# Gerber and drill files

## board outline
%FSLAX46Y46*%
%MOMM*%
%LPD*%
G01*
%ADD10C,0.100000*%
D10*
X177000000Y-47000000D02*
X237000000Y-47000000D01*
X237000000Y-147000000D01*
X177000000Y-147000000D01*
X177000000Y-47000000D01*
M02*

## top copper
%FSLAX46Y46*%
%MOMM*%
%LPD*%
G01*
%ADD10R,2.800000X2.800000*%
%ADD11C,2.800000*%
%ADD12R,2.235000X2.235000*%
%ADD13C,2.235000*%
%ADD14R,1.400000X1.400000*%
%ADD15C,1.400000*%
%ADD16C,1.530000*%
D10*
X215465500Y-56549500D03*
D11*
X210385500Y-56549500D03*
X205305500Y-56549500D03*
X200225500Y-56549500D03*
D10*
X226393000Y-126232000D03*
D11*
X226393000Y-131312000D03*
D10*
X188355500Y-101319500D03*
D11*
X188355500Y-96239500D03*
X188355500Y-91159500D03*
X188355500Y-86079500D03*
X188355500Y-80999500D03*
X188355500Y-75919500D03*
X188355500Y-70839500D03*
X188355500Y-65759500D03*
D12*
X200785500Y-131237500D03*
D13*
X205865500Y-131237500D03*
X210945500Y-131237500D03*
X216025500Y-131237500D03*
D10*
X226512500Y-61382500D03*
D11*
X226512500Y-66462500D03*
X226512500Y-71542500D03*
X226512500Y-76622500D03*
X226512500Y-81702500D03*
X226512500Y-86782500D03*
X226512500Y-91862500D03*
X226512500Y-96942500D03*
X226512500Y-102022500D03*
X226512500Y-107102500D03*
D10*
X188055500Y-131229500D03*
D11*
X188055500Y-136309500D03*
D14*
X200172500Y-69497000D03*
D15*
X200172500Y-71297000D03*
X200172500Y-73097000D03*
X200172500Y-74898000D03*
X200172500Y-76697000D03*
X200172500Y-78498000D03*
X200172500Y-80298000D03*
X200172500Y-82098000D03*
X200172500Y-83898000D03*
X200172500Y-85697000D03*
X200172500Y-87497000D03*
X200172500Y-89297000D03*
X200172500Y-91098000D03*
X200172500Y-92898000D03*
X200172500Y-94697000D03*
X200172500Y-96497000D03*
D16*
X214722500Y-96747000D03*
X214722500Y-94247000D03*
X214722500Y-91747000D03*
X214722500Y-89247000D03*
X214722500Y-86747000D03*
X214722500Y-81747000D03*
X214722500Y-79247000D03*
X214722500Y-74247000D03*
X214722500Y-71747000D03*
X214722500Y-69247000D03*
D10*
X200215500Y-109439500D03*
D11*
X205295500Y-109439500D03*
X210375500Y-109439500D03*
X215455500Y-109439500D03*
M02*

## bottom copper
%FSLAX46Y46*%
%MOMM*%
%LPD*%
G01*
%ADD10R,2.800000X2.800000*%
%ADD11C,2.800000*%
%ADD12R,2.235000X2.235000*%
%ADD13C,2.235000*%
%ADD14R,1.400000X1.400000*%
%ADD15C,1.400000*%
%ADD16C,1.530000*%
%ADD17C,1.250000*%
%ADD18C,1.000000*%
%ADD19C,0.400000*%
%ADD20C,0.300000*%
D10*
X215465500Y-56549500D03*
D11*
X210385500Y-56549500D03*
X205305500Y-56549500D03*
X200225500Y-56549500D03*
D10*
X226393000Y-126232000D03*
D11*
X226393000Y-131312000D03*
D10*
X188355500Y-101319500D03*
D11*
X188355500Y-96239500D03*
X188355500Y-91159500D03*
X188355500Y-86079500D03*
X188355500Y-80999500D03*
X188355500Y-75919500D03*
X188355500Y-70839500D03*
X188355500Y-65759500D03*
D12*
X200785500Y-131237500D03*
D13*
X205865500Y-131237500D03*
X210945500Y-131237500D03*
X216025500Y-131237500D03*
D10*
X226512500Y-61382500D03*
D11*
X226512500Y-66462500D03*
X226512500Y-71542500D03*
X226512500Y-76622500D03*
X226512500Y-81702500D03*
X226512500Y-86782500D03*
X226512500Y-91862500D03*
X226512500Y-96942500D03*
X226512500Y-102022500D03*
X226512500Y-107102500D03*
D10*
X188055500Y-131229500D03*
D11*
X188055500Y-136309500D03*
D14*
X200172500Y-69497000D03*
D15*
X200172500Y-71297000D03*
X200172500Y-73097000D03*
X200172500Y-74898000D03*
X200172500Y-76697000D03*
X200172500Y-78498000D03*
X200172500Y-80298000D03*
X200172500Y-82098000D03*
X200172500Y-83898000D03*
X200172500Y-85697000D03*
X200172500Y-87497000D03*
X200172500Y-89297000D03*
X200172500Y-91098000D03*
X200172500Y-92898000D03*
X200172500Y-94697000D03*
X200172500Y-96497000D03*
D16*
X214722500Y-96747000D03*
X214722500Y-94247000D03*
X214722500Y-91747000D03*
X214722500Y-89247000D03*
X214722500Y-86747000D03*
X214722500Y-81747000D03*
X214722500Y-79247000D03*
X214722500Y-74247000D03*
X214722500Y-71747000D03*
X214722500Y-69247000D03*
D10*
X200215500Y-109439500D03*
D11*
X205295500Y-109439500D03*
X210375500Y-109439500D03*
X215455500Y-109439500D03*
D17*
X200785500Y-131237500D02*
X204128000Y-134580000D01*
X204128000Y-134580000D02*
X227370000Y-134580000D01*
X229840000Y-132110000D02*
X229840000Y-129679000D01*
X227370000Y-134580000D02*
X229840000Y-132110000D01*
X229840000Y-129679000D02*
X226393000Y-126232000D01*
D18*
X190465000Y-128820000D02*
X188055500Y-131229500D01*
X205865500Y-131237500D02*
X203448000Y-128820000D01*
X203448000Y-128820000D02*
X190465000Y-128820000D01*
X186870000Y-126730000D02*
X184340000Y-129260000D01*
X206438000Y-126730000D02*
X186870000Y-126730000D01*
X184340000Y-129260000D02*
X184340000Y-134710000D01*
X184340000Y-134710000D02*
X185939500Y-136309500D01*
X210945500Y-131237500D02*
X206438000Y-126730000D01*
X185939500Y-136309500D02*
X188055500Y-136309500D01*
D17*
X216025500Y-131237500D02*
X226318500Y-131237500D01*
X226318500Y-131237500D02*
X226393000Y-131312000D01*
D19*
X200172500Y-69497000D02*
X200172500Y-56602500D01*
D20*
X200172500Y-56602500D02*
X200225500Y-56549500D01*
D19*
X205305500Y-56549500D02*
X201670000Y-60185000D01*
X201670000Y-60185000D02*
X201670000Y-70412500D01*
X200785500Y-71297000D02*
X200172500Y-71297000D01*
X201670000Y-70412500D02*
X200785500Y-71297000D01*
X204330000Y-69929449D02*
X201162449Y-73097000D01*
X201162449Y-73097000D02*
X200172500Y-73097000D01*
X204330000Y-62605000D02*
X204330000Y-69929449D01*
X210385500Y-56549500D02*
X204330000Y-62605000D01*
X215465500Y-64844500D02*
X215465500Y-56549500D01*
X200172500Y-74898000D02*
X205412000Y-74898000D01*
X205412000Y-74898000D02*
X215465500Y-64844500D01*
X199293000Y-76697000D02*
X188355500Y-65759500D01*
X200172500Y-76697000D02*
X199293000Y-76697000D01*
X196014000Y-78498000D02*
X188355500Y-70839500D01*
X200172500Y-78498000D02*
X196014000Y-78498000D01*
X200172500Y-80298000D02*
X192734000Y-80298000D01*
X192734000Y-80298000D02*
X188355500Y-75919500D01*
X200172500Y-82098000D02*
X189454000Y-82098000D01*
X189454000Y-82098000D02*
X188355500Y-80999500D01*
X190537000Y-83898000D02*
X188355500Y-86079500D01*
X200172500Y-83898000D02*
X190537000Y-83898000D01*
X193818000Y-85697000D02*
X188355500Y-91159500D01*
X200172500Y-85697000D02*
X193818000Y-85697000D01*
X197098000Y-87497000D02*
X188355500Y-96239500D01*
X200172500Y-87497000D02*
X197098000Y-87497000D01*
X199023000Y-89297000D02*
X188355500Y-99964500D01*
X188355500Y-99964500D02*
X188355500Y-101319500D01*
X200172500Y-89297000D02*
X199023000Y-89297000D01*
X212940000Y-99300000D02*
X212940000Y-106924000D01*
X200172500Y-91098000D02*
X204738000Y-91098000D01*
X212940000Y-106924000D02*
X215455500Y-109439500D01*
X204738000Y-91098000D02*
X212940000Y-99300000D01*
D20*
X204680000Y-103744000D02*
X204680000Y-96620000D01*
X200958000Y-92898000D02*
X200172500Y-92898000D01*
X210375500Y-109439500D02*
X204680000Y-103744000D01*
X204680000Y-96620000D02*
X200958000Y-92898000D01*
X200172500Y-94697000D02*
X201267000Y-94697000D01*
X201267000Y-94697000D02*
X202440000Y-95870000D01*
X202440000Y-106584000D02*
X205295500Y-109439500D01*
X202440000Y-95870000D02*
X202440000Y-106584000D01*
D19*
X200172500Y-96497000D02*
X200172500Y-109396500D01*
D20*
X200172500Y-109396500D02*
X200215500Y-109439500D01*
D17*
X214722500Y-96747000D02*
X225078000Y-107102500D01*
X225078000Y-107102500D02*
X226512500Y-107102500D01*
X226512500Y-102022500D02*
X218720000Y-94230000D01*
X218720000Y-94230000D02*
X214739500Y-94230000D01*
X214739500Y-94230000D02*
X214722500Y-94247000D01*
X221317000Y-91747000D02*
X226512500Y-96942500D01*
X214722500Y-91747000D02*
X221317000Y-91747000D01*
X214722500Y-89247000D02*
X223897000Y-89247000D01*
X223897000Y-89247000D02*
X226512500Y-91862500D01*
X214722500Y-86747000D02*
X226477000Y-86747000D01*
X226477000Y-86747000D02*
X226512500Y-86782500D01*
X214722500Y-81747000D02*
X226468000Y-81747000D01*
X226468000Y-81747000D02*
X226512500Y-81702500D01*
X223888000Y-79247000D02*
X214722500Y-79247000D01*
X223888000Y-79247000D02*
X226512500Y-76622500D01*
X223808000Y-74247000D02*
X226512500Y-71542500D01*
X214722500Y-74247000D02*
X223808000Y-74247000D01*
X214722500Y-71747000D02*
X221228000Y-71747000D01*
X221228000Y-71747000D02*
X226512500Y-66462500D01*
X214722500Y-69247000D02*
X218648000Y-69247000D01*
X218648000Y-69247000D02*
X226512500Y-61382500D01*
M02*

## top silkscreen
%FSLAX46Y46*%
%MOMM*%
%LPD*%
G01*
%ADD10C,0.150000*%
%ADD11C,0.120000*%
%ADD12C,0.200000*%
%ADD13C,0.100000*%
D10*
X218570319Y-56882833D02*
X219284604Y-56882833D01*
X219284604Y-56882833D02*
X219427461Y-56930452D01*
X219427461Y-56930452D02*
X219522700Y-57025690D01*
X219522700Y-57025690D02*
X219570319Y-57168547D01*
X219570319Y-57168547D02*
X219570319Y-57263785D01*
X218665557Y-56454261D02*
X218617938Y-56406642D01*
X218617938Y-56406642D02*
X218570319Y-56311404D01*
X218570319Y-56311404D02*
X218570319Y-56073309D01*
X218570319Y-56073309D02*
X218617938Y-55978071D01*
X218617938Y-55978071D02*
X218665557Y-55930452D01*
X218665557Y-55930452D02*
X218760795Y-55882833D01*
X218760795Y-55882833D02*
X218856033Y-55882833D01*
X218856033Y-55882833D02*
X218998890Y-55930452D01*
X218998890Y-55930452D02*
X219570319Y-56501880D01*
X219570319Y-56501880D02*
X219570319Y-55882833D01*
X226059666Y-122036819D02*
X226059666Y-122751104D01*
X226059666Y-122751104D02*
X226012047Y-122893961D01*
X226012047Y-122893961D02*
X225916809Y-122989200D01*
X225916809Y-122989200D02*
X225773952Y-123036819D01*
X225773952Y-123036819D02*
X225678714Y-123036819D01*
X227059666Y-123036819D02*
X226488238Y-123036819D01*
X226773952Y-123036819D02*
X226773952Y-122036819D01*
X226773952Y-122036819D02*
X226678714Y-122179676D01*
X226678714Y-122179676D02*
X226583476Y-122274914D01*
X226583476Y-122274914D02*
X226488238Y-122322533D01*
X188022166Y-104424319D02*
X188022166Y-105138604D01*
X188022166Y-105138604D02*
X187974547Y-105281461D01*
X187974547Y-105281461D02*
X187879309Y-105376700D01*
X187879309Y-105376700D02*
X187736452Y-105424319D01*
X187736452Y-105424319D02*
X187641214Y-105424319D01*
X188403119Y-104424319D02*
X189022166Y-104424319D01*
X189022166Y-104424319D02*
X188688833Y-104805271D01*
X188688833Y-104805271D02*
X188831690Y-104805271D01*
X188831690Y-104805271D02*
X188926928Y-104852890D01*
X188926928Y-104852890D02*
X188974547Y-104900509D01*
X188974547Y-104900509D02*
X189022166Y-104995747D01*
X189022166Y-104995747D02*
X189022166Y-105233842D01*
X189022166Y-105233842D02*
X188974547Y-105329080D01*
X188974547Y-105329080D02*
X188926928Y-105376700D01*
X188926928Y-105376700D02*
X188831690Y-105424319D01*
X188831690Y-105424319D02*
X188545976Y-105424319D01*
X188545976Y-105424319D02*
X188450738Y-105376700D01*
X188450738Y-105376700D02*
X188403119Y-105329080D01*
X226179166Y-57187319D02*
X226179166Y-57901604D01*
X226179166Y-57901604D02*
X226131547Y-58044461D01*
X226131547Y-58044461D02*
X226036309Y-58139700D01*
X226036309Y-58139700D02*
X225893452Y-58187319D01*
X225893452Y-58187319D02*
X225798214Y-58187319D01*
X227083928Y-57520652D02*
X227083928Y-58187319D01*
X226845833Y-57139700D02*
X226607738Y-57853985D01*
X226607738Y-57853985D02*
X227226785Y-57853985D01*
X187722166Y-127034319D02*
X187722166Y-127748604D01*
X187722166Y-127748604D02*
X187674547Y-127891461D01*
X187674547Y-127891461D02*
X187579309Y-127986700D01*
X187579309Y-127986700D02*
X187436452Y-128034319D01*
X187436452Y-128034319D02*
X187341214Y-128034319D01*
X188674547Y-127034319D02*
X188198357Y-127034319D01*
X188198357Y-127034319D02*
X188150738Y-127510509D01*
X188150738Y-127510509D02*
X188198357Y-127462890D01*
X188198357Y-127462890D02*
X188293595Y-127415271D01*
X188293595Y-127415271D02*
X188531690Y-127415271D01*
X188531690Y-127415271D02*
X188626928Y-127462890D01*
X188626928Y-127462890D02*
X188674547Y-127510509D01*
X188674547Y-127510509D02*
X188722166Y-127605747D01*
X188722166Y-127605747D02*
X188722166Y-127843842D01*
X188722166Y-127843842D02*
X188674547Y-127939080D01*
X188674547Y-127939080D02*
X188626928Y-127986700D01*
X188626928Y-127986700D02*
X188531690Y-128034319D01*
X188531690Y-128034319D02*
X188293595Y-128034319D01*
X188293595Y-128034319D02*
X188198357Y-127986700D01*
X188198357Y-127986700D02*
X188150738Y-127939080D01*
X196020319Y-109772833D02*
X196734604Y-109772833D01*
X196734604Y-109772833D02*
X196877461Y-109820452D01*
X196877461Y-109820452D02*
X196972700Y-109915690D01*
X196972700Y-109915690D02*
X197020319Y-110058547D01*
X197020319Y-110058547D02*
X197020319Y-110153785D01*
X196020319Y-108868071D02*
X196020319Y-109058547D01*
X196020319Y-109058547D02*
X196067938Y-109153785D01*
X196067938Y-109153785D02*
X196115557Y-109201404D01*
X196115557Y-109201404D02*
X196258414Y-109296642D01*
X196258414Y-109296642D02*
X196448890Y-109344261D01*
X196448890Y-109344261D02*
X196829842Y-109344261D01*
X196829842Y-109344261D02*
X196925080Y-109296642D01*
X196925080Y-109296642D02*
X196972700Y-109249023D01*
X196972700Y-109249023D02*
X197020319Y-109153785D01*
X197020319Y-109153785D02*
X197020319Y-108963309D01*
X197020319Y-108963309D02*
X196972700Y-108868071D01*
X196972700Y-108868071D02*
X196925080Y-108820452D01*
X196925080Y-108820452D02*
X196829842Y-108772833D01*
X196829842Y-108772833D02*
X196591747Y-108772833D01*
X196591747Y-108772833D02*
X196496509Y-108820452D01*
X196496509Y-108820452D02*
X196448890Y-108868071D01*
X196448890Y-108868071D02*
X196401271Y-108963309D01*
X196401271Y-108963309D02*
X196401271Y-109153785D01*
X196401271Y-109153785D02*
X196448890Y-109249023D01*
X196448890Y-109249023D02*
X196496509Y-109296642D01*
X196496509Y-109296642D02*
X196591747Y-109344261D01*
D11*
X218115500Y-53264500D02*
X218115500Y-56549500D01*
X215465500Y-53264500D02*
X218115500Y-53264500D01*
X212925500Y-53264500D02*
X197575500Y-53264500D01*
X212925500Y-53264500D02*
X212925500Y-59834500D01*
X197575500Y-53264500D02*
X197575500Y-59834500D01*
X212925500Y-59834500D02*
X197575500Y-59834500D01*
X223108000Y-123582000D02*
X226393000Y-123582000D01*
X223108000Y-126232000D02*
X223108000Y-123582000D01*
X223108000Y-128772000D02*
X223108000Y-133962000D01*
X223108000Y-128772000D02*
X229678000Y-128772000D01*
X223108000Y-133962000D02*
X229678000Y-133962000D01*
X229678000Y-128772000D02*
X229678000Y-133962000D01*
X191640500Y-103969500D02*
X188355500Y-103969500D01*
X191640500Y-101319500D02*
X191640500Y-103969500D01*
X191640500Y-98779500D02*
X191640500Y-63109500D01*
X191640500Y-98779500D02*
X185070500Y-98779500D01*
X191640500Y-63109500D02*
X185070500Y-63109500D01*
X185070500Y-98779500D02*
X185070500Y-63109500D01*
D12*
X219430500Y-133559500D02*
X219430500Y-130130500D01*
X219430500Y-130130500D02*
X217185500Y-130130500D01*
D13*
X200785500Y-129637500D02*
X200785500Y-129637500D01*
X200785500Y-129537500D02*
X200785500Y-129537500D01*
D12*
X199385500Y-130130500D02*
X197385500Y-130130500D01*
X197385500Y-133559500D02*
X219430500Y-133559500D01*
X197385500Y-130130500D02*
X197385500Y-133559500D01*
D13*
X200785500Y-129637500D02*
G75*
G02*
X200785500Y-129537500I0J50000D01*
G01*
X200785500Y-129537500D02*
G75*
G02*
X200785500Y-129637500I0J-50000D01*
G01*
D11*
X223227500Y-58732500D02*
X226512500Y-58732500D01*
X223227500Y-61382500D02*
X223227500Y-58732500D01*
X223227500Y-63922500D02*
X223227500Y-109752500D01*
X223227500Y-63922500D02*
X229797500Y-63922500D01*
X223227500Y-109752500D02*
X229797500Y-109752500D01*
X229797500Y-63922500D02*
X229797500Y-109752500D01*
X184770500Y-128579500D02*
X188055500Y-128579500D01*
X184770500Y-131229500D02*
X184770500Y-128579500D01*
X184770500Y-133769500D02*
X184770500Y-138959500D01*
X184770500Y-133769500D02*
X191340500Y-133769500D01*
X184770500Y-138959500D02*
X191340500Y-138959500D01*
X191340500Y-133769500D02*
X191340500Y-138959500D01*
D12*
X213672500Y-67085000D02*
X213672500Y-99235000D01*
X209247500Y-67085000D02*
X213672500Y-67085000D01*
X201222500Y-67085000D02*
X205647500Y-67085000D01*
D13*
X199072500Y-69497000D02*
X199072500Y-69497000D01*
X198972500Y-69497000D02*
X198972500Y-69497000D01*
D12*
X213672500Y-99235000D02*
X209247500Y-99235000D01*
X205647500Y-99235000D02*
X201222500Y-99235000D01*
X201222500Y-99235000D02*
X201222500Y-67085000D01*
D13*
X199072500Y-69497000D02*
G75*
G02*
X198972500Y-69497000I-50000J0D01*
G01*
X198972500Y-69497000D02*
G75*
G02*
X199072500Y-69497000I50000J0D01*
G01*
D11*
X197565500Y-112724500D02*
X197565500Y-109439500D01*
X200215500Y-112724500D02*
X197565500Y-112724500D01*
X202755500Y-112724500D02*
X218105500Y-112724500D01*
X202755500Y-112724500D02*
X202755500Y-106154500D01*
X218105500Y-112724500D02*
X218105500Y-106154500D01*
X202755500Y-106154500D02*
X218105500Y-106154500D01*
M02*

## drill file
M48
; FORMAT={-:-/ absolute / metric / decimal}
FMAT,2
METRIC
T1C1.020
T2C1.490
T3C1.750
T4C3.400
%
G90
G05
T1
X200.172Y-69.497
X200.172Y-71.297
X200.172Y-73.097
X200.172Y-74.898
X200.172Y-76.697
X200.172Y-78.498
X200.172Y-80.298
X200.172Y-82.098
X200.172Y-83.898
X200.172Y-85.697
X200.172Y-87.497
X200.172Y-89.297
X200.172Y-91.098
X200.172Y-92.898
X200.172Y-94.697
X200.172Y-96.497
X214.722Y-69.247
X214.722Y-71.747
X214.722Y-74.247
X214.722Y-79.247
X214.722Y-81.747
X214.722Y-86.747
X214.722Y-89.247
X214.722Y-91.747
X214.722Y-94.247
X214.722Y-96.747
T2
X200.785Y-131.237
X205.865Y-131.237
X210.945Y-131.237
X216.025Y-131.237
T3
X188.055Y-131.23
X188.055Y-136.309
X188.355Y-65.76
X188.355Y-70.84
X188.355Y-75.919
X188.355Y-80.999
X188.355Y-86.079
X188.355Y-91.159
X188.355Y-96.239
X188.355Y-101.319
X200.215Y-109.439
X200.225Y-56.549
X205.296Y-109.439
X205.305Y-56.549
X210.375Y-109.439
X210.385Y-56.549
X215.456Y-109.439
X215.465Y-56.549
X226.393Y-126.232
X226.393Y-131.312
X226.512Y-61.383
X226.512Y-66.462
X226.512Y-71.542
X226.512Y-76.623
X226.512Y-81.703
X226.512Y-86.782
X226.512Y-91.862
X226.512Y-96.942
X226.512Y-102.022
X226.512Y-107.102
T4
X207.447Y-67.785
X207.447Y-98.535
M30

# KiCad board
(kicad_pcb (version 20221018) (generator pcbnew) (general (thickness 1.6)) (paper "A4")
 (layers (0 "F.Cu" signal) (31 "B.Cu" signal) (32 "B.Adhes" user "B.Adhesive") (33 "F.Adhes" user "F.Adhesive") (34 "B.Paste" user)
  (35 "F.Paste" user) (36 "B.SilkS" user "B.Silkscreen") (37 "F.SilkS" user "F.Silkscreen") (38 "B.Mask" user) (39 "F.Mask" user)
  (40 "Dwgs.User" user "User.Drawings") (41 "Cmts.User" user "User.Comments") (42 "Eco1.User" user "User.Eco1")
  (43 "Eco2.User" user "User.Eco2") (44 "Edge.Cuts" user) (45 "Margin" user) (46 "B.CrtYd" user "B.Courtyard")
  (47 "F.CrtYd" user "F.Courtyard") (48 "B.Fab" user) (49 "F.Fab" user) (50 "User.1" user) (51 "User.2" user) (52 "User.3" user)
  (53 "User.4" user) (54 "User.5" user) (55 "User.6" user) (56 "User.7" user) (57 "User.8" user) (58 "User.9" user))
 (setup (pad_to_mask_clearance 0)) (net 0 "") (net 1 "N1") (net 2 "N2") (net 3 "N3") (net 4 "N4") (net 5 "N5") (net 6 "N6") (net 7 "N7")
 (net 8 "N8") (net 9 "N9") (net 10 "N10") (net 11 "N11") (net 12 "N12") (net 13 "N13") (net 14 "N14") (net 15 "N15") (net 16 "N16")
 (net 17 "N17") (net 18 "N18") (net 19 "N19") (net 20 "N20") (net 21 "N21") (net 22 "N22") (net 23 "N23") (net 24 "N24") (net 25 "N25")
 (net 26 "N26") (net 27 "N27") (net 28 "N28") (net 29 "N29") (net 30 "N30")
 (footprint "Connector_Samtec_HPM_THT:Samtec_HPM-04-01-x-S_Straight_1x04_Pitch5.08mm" (layer "F.Cu") (at 215.4655 56.5495 -90)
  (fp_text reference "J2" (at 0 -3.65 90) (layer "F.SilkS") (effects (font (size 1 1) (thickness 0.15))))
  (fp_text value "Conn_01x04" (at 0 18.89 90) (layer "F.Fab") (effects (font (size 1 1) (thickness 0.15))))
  (fp_line (start -3.285 -2.65) (end 0 -2.65) (stroke (width 0.12) (type solid)) (layer "F.SilkS"))
  (fp_line (start -3.285 0) (end -3.285 -2.65) (stroke (width 0.12) (type solid)) (layer "F.SilkS"))
  (fp_line (start -3.285 2.54) (end -3.285 17.89) (stroke (width 0.12) (type solid)) (layer "F.SilkS"))
  (fp_line (start -3.285 2.54) (end 3.285 2.54) (stroke (width 0.12) (type solid)) (layer "F.SilkS"))
  (fp_line (start -3.285 17.89) (end 3.285 17.89) (stroke (width 0.12) (type solid)) (layer "F.SilkS"))
  (fp_line (start 3.285 2.54) (end 3.285 17.89) (stroke (width 0.12) (type solid)) (layer "F.SilkS"))
  (pad "1" thru_hole rect (at 0 0 270) (size 2.8 2.8) (drill 1.75) (layers "*.Cu" "*.Mask") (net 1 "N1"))
  (pad "2" thru_hole circle (at 0 5.08 270) (size 2.8 2.8) (drill 1.75) (layers "*.Cu" "*.Mask") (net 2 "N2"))
  (pad "3" thru_hole circle (at 0 10.16 270) (size 2.8 2.8) (drill 1.75) (layers "*.Cu" "*.Mask") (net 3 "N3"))
  (pad "4" thru_hole circle (at 0 15.24 270) (size 2.8 2.8) (drill 1.75) (layers "*.Cu" "*.Mask") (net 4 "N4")))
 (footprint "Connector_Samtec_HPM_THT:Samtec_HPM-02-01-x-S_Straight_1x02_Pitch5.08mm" (layer "F.Cu") (at 226.393 126.232)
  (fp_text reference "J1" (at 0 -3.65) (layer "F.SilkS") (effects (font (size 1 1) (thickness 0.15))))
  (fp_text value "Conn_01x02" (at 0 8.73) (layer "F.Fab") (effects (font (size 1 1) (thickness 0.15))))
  (fp_line (start -3.285 -2.65) (end 0 -2.65) (stroke (width 0.12) (type solid)) (layer "F.SilkS"))
  (fp_line (start -3.285 0) (end -3.285 -2.65) (stroke (width 0.12) (type solid)) (layer "F.SilkS"))
  (fp_line (start -3.285 2.54) (end -3.285 7.73) (stroke (width 0.12) (type solid)) (layer "F.SilkS"))
  (fp_line (start -3.285 2.54) (end 3.285 2.54) (stroke (width 0.12) (type solid)) (layer "F.SilkS"))
  (fp_line (start -3.285 7.73) (end 3.285 7.73) (stroke (width 0.12) (type solid)) (layer "F.SilkS"))
  (fp_line (start 3.285 2.54) (end 3.285 7.73) (stroke (width 0.12) (type solid)) (layer "F.SilkS"))
  (pad "1" thru_hole rect (at 0 0) (size 2.8 2.8) (drill 1.75) (layers "*.Cu" "*.Mask") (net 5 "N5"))
  (pad "2" thru_hole circle (at 0 5.08) (size 2.8 2.8) (drill 1.75) (layers "*.Cu" "*.Mask") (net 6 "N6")))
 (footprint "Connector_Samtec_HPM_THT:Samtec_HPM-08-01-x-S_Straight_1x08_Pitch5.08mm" (layer "F.Cu") (at 188.3555 101.3195 180)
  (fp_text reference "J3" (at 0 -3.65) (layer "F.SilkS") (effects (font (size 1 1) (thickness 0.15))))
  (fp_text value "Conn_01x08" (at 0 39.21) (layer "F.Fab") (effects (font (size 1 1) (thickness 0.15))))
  (fp_line (start -3.285 -2.65) (end 0 -2.65) (stroke (width 0.12) (type solid)) (layer "F.SilkS"))
  (fp_line (start -3.285 0) (end -3.285 -2.65) (stroke (width 0.12) (type solid)) (layer "F.SilkS"))
  (fp_line (start -3.285 2.54) (end -3.285 38.21) (stroke (width 0.12) (type solid)) (layer "F.SilkS"))
  (fp_line (start -3.285 2.54) (end 3.285 2.54) (stroke (width 0.12) (type solid)) (layer "F.SilkS"))
  (fp_line (start -3.285 38.21) (end 3.285 38.21) (stroke (width 0.12) (type solid)) (layer "F.SilkS"))
  (fp_line (start 3.285 2.54) (end 3.285 38.21) (stroke (width 0.12) (type solid)) (layer "F.SilkS"))
  (pad "1" thru_hole rect (at 0 0 180) (size 2.8 2.8) (drill 1.75) (layers "*.Cu" "*.Mask") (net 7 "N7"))
  (pad "2" thru_hole circle (at 0 5.08 180) (size 2.8 2.8) (drill 1.75) (layers "*.Cu" "*.Mask") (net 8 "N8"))
  (pad "3" thru_hole circle (at 0 10.16 180) (size 2.8 2.8) (drill 1.75) (layers "*.Cu" "*.Mask") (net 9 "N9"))
  (pad "4" thru_hole circle (at 0 15.24 180) (size 2.8 2.8) (drill 1.75) (layers "*.Cu" "*.Mask") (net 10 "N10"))
  (pad "5" thru_hole circle (at 0 20.32 180) (size 2.8 2.8) (drill 1.75) (layers "*.Cu" "*.Mask") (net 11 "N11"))
  (pad "6" thru_hole circle (at 0 25.4 180) (size 2.8 2.8) (drill 1.75) (layers "*.Cu" "*.Mask") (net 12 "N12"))
  (pad "7" thru_hole circle (at 0 30.48 180) (size 2.8 2.8) (drill 1.75) (layers "*.Cu" "*.Mask") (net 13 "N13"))
  (pad "8" thru_hole circle (at 0 35.56 180) (size 2.8 2.8) (drill 1.75) (layers "*.Cu" "*.Mask") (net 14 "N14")))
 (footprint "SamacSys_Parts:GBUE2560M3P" (layer "F.Cu") (at 200.7855 131.2375 180)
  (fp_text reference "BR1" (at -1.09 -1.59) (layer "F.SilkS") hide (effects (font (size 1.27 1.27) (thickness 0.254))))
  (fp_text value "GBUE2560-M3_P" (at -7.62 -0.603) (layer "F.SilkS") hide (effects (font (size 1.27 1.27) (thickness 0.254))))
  (fp_line (start -18.645 -2.322) (end -18.645 1.107) (stroke (width 0.2) (type solid)) (layer "F.SilkS"))
  (fp_line (start -18.645 1.107) (end -16.4 1.107) (stroke (width 0.2) (type solid)) (layer "F.SilkS"))
  (fp_line (start 0 1.6) (end 0 1.6) (stroke (width 0.1) (type solid)) (layer "F.SilkS"))
  (fp_line (start 0 1.7) (end 0 1.7) (stroke (width 0.1) (type solid)) (layer "F.SilkS"))
  (fp_line (start 1.4 1.107) (end 3.4 1.107) (stroke (width 0.2) (type solid)) (layer "F.SilkS"))
  (fp_line (start 3.4 -2.322) (end -18.645 -2.322) (stroke (width 0.2) (type solid)) (layer "F.SilkS"))
  (fp_line (start 3.4 1.107) (end 3.4 -2.322) (stroke (width 0.2) (type solid)) (layer "F.SilkS"))
  (fp_arc (start 0 1.6) (mid 0.05 1.65) (end 0 1.7) (stroke (width 0.1) (type solid)) (layer "F.SilkS"))
  (fp_arc (start 0 1.7) (mid -0.05 1.65) (end 0 1.6) (stroke (width 0.1) (type solid)) (layer "F.SilkS"))
  (pad "1" thru_hole rect (at 0 0 180) (size 2.235 2.235) (drill 1.49) (layers "*.Cu" "*.Mask") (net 5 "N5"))
  (pad "2" thru_hole circle (at -5.08 0 180) (size 2.235 2.235) (drill 1.49) (layers "*.Cu" "*.Mask") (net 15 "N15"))
  (pad "3" thru_hole circle (at -10.16 0 180) (size 2.235 2.235) (drill 1.49) (layers "*.Cu" "*.Mask") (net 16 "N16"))
  (pad "4" thru_hole circle (at -15.24 0 180) (size 2.235 2.235) (drill 1.49) (layers "*.Cu" "*.Mask") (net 6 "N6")))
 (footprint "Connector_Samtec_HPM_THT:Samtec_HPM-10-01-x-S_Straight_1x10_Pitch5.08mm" (layer "F.Cu") (at 226.5125 61.3825)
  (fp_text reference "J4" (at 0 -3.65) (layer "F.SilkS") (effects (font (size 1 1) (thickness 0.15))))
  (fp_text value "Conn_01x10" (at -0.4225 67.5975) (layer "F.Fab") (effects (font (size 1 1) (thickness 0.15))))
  (fp_line (start -3.285 -2.65) (end 0 -2.65) (stroke (width 0.12) (type solid)) (layer "F.SilkS"))
  (fp_line (start -3.285 0) (end -3.285 -2.65) (stroke (width 0.12) (type solid)) (layer "F.SilkS"))
  (fp_line (start -3.285 2.54) (end -3.285 48.37) (stroke (width 0.12) (type solid)) (layer "F.SilkS"))
  (fp_line (start -3.285 2.54) (end 3.285 2.54) (stroke (width 0.12) (type solid)) (layer "F.SilkS"))
  (fp_line (start -3.285 48.37) (end 3.285 48.37) (stroke (width 0.12) (type solid)) (layer "F.SilkS"))
  (fp_line (start 3.285 2.54) (end 3.285 48.37) (stroke (width 0.12) (type solid)) (layer "F.SilkS"))
  (pad "1" thru_hole rect (at 0 0) (size 2.8 2.8) (drill 1.75) (layers "*.Cu" "*.Mask") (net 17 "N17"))
  (pad "2" thru_hole circle (at 0 5.08) (size 2.8 2.8) (drill 1.75) (layers "*.Cu" "*.Mask") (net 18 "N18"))
  (pad "3" thru_hole circle (at 0 10.16) (size 2.8 2.8) (drill 1.75) (layers "*.Cu" "*.Mask") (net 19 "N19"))
  (pad "4" thru_hole circle (at 0 15.24) (size 2.8 2.8) (drill 1.75) (layers "*.Cu" "*.Mask") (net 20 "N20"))
  (pad "5" thru_hole circle (at 0 20.32) (size 2.8 2.8) (drill 1.75) (layers "*.Cu" "*.Mask") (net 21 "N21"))
  (pad "6" thru_hole circle (at 0 25.4) (size 2.8 2.8) (drill 1.75) (layers "*.Cu" "*.Mask") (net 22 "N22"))
  (pad "7" thru_hole circle (at 0 30.48) (size 2.8 2.8) (drill 1.75) (layers "*.Cu" "*.Mask") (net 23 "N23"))
  (pad "8" thru_hole circle (at 0 35.56) (size 2.8 2.8) (drill 1.75) (layers "*.Cu" "*.Mask") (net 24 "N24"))
  (pad "9" thru_hole circle (at 0 40.64) (size 2.8 2.8) (drill 1.75) (layers "*.Cu" "*.Mask") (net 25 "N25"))
  (pad "10" thru_hole circle (at 0 45.72) (size 2.8 2.8) (drill 1.75) (layers "*.Cu" "*.Mask") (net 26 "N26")))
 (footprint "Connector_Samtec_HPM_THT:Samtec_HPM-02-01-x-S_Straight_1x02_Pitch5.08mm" (layer "F.Cu") (at 188.0555 131.2295)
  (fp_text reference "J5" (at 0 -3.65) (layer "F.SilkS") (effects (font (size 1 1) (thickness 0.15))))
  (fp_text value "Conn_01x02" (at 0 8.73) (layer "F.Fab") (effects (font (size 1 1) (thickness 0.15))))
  (fp_line (start -3.285 -2.65) (end 0 -2.65) (stroke (width 0.12) (type solid)) (layer "F.SilkS"))
  (fp_line (start -3.285 0) (end -3.285 -2.65) (stroke (width 0.12) (type solid)) (layer "F.SilkS"))
  (fp_line (start -3.285 2.54) (end -3.285 7.73) (stroke (width 0.12) (type solid)) (layer "F.SilkS"))
  (fp_line (start -3.285 2.54) (end 3.285 2.54) (stroke (width 0.12) (type solid)) (layer "F.SilkS"))
  (fp_line (start -3.285 7.73) (end 3.285 7.73) (stroke (width 0.12) (type solid)) (layer "F.SilkS"))
  (fp_line (start 3.285 2.54) (end 3.285 7.73) (stroke (width 0.12) (type solid)) (layer "F.SilkS"))
  (pad "1" thru_hole rect (at 0 0) (size 2.8 2.8) (drill 1.75) (layers "*.Cu" "*.Mask") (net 15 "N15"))
  (pad "2" thru_hole circle (at 0 5.08) (size 2.8 2.8) (drill 1.75) (layers "*.Cu" "*.Mask") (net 16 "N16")))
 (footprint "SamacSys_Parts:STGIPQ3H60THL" (layer "F.Cu") (at 200.1725 69.497 -90)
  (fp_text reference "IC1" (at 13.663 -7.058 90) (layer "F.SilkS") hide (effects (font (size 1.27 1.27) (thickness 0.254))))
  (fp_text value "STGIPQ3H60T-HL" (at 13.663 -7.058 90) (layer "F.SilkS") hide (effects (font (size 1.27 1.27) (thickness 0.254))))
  (fp_line (start -2.412 -13.5) (end 29.738 -13.5) (stroke (width 0.2) (type solid)) (layer "F.SilkS"))
  (fp_line (start -2.412 -9.075) (end -2.412 -13.5) (stroke (width 0.2) (type solid)) (layer "F.SilkS"))
  (fp_line (start -2.412 -1.05) (end -2.412 -5.475) (stroke (width 0.2) (type solid)) (layer "F.SilkS"))
  (fp_line (start 0 1.1) (end 0 1.1) (stroke (width 0.1) (type solid)) (layer "F.SilkS"))
  (fp_line (start 0 1.2) (end 0 1.2) (stroke (width 0.1) (type solid)) (layer "F.SilkS"))
  (fp_line (start 29.738 -13.5) (end 29.738 -9.075) (stroke (width 0.2) (type solid)) (layer "F.SilkS"))
  (fp_line (start 29.738 -5.475) (end 29.738 -1.05) (stroke (width 0.2) (type solid)) (layer "F.SilkS"))
  (fp_line (start 29.738 -1.05) (end -2.412 -1.05) (stroke (width 0.2) (type solid)) (layer "F.SilkS"))
  (fp_arc (start 0 1.1) (mid 0.05 1.15) (end 0 1.2) (stroke (width 0.1) (type solid)) (layer "F.SilkS"))
  (fp_arc (start 0 1.2) (mid -0.05 1.15) (end 0 1.1) (stroke (width 0.1) (type solid)) (layer "F.SilkS"))
  (pad "" np_thru_hole circle (at -1.712 -7.275 270) (size 3.4 3.4) (drill 3.4) (layers "*.Cu" "*.Mask"))
  (pad "" np_thru_hole circle (at 29.038 -7.275 270) (size 3.4 3.4) (drill 3.4) (layers "*.Cu" "*.Mask"))
  (pad "1" thru_hole rect (at 0 0 270) (size 1.4 1.4) (drill 1.02) (layers "*.Cu" "*.Mask") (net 4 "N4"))
  (pad "2" thru_hole circle (at 1.8 0 270) (size 1.4 1.4) (drill 1.02) (layers "*.Cu" "*.Mask") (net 3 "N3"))
  (pad "3" thru_hole circle (at 3.6 0 270) (size 1.4 1.4) (drill 1.02) (layers "*.Cu" "*.Mask") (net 2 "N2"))
  (pad "4" thru_hole circle (at 5.401 0 270) (size 1.4 1.4) (drill 1.02) (layers "*.Cu" "*.Mask") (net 1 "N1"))
  (pad "5" thru_hole circle (at 7.2 0 270) (size 1.4 1.4) (drill 1.02) (layers "*.Cu" "*.Mask") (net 14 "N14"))
  (pad "6" thru_hole circle (at 9.001 0 270) (size 1.4 1.4) (drill 1.02) (layers "*.Cu" "*.Mask") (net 13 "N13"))
  (pad "7" thru_hole circle (at 10.801 0 270) (size 1.4 1.4) (drill 1.02) (layers "*.Cu" "*.Mask") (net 12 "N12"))
  (pad "8" thru_hole circle (at 12.601 0 270) (size 1.4 1.4) (drill 1.02) (layers "*.Cu" "*.Mask") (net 11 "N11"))
  (pad "9" thru_hole circle (at 14.401 0 270) (size 1.4 1.4) (drill 1.02) (layers "*.Cu" "*.Mask") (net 10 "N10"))
  (pad "10" thru_hole circle (at 16.2 0 270) (size 1.4 1.4) (drill 1.02) (layers "*.Cu" "*.Mask") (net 9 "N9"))
  (pad "11" thru_hole circle (at 18 0 270) (size 1.4 1.4) (drill 1.02) (layers "*.Cu" "*.Mask") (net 8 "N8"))
  (pad "12" thru_hole circle (at 19.8 0 270) (size 1.4 1.4) (drill 1.02) (layers "*.Cu" "*.Mask") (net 7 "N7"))
  (pad "13" thru_hole circle (at 21.601 0 270) (size 1.4 1.4) (drill 1.02) (layers "*.Cu" "*.Mask") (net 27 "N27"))
  (pad "14" thru_hole circle (at 23.401 0 270) (size 1.4 1.4) (drill 1.02) (layers "*.Cu" "*.Mask") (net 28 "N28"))
  (pad "15" thru_hole circle (at 25.2 0 270) (size 1.4 1.4) (drill 1.02) (layers "*.Cu" "*.Mask") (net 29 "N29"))
  (pad "16" thru_hole circle (at 27 0 270) (size 1.4 1.4) (drill 1.02) (layers "*.Cu" "*.Mask") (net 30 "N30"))
  (pad "17" thru_hole circle (at 27.25 -14.55 270) (size 1.53 1.53) (drill 1.02) (layers "*.Cu" "*.Mask") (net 26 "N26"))
  (pad "18" thru_hole circle (at 24.75 -14.55 270) (size 1.53 1.53) (drill 1.02) (layers "*.Cu" "*.Mask") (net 25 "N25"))
  (pad "19" thru_hole circle (at 22.25 -14.55 270) (size 1.53 1.53) (drill 1.02) (layers "*.Cu" "*.Mask") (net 24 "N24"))
  (pad "20" thru_hole circle (at 19.75 -14.55 270) (size 1.53 1.53) (drill 1.02) (layers "*.Cu" "*.Mask") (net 23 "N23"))
  (pad "21" thru_hole circle (at 17.25 -14.55 270) (size 1.53 1.53) (drill 1.02) (layers "*.Cu" "*.Mask") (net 22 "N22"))
  (pad "22" thru_hole circle (at 12.25 -14.55 270) (size 1.53 1.53) (drill 1.02) (layers "*.Cu" "*.Mask") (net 21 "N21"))
  (pad "23" thru_hole circle (at 9.75 -14.55 270) (size 1.53 1.53) (drill 1.02) (layers "*.Cu" "*.Mask") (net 20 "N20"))
  (pad "24" thru_hole circle (at 4.75 -14.55 270) (size 1.53 1.53) (drill 1.02) (layers "*.Cu" "*.Mask") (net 19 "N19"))
  (pad "25" thru_hole circle (at 2.25 -14.55 270) (size 1.53 1.53) (drill 1.02) (layers "*.Cu" "*.Mask") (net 18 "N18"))
  (pad "26" thru_hole circle (at -0.25 -14.55 270) (size 1.53 1.53) (drill 1.02) (layers "*.Cu" "*.Mask") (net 17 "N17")))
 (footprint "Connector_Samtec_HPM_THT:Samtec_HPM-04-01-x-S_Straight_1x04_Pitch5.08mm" (layer "F.Cu") (at 200.2155 109.4395 90)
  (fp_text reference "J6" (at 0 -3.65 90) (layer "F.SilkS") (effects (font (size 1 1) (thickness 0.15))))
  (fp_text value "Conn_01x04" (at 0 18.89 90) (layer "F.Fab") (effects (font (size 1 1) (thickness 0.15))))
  (fp_line (start -3.285 -2.65) (end 0 -2.65) (stroke (width 0.12) (type solid)) (layer "F.SilkS"))
  (fp_line (start -3.285 0) (end -3.285 -2.65) (stroke (width 0.12) (type solid)) (layer "F.SilkS"))
  (fp_line (start -3.285 2.54) (end -3.285 17.89) (stroke (width 0.12) (type solid)) (layer "F.SilkS"))
  (fp_line (start -3.285 2.54) (end 3.285 2.54) (stroke (width 0.12) (type solid)) (layer "F.SilkS"))
  (fp_line (start -3.285 17.89) (end 3.285 17.89) (stroke (width 0.12) (type solid)) (layer "F.SilkS"))
  (fp_line (start 3.285 2.54) (end 3.285 17.89) (stroke (width 0.12) (type solid)) (layer "F.SilkS"))
  (pad "1" thru_hole rect (at 0 0 90) (size 2.8 2.8) (drill 1.75) (layers "*.Cu" "*.Mask") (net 30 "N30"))
  (pad "2" thru_hole circle (at 0 5.08 90) (size 2.8 2.8) (drill 1.75) (layers "*.Cu" "*.Mask") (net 29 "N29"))
  (pad "3" thru_hole circle (at 0 10.16 90) (size 2.8 2.8) (drill 1.75) (layers "*.Cu" "*.Mask") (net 28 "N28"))
  (pad "4" thru_hole circle (at 0 15.24 90) (size 2.8 2.8) (drill 1.75) (layers "*.Cu" "*.Mask") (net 27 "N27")))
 (gr_rect (start 177 47) (end 237 147) (stroke (width 0.1) (type default)) (fill none) (layer "Edge.Cuts"))
 (segment (start 200.7855 131.2375) (end 204.128 134.58) (width 1.25) (layer "B.Cu") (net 5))
 (segment (start 204.128 134.58) (end 227.37 134.58) (width 1.25) (layer "B.Cu") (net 5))
 (segment (start 229.84 132.11) (end 229.84 129.679) (width 1.25) (layer "B.Cu") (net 5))
 (segment (start 227.37 134.58) (end 229.84 132.11) (width 1.25) (layer "B.Cu") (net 5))
 (segment (start 229.84 129.679) (end 226.393 126.232) (width 1.25) (layer "B.Cu") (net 5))
 (segment (start 190.465 128.82) (end 188.0555 131.2295) (width 1) (layer "B.Cu") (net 15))
 (segment (start 205.8655 131.2375) (end 203.448 128.82) (width 1) (layer "B.Cu") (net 15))
 (segment (start 203.448 128.82) (end 190.465 128.82) (width 1) (layer "B.Cu") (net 15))
 (segment (start 186.87 126.73) (end 184.34 129.26) (width 1) (layer "B.Cu") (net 16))
 (segment (start 206.438 126.73) (end 186.87 126.73) (width 1) (layer "B.Cu") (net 16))
 (segment (start 184.34 129.26) (end 184.34 134.71) (width 1) (layer "B.Cu") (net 16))
 (segment (start 184.34 134.71) (end 185.9395 136.3095) (width 1) (layer "B.Cu") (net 16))
 (segment (start 210.9455 131.2375) (end 206.438 126.73) (width 1) (layer "B.Cu") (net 16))
 (segment (start 185.9395 136.3095) (end 188.0555 136.3095) (width 1) (layer "B.Cu") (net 16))
 (segment (start 216.0255 131.2375) (end 226.3185 131.2375) (width 1.25) (layer "B.Cu") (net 6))
 (segment (start 226.3185 131.2375) (end 226.393 131.312) (width 1.25) (layer "B.Cu") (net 6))
 (segment (start 200.1725 69.497) (end 200.1725 56.6025) (width 0.4) (layer "B.Cu") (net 4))
 (segment (start 200.1725 56.6025) (end 200.2255 56.5495) (width 0.3) (layer "B.Cu") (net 4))
 (segment (start 205.3055 56.5495) (end 201.67 60.185) (width 0.4) (layer "B.Cu") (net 3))
 (segment (start 201.67 60.185) (end 201.67 70.4125) (width 0.4) (layer "B.Cu") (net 3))
 (segment (start 200.7855 71.297) (end 200.1725 71.297) (width 0.4) (layer "B.Cu") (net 3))
 (segment (start 201.67 70.4125) (end 200.7855 71.297) (width 0.4) (layer "B.Cu") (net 3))
 (segment (start 204.33 69.929449) (end 201.162449 73.097) (width 0.4) (layer "B.Cu") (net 2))
 (segment (start 201.162449 73.097) (end 200.1725 73.097) (width 0.4) (layer "B.Cu") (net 2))
 (segment (start 204.33 62.605) (end 204.33 69.929449) (width 0.4) (layer "B.Cu") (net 2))
 (segment (start 210.3855 56.5495) (end 204.33 62.605) (width 0.4) (layer "B.Cu") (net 2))
 (segment (start 215.4655 64.8445) (end 215.4655 56.5495) (width 0.4) (layer "B.Cu") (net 1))
 (segment (start 200.1725 74.898) (end 205.412 74.898) (width 0.4) (layer "B.Cu") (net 1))
 (segment (start 205.412 74.898) (end 215.4655 64.8445) (width 0.4) (layer "B.Cu") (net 1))
 (segment (start 199.293 76.697) (end 188.3555 65.7595) (width 0.4) (layer "B.Cu") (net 14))
 (segment (start 200.1725 76.697) (end 199.293 76.697) (width 0.4) (layer "B.Cu") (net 14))
 (segment (start 196.014 78.498) (end 188.3555 70.8395) (width 0.4) (layer "B.Cu") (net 13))
 (segment (start 200.1725 78.498) (end 196.014 78.498) (width 0.4) (layer "B.Cu") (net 13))
 (segment (start 200.1725 80.298) (end 192.734 80.298) (width 0.4) (layer "B.Cu") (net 12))
 (segment (start 192.734 80.298) (end 188.3555 75.9195) (width 0.4) (layer "B.Cu") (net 12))
 (segment (start 200.1725 82.098) (end 189.454 82.098) (width 0.4) (layer "B.Cu") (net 11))
 (segment (start 189.454 82.098) (end 188.3555 80.9995) (width 0.4) (layer "B.Cu") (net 11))
 (segment (start 190.537 83.898) (end 188.3555 86.0795) (width 0.4) (layer "B.Cu") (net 10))
 (segment (start 200.1725 83.898) (end 190.537 83.898) (width 0.4) (layer "B.Cu") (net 10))
 (segment (start 193.818 85.697) (end 188.3555 91.1595) (width 0.4) (layer "B.Cu") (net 9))
 (segment (start 200.1725 85.697) (end 193.818 85.697) (width 0.4) (layer "B.Cu") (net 9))
 (segment (start 197.098 87.497) (end 188.3555 96.2395) (width 0.4) (layer "B.Cu") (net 8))
 (segment (start 200.1725 87.497) (end 197.098 87.497) (width 0.4) (layer "B.Cu") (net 8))
 (segment (start 199.023 89.297) (end 188.3555 99.9645) (width 0.4) (layer "B.Cu") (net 7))
 (segment (start 188.3555 99.9645) (end 188.3555 101.3195) (width 0.4) (layer "B.Cu") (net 7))
 (segment (start 200.1725 89.297) (end 199.023 89.297) (width 0.4) (layer "B.Cu") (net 7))
 (segment (start 212.94 99.3) (end 212.94 106.924) (width 0.4) (layer "B.Cu") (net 27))
 (segment (start 200.1725 91.098) (end 204.738 91.098) (width 0.4) (layer "B.Cu") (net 27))
 (segment (start 212.94 106.924) (end 215.4555 109.4395) (width 0.4) (layer "B.Cu") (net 27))
 (segment (start 204.738 91.098) (end 212.94 99.3) (width 0.4) (layer "B.Cu") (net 27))
 (segment (start 204.68 103.744) (end 204.68 96.62) (width 0.3) (layer "B.Cu") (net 28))
 (segment (start 200.958 92.898) (end 200.1725 92.898) (width 0.3) (layer "B.Cu") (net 28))
 (segment (start 210.3755 109.4395) (end 204.68 103.744) (width 0.3) (layer "B.Cu") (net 28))
 (segment (start 204.68 96.62) (end 200.958 92.898) (width 0.3) (layer "B.Cu") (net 28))
 (segment (start 200.1725 94.697) (end 201.267 94.697) (width 0.3) (layer "B.Cu") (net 29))
 (segment (start 201.267 94.697) (end 202.44 95.87) (width 0.3) (layer "B.Cu") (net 29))
 (segment (start 202.44 106.584) (end 205.2955 109.4395) (width 0.3) (layer "B.Cu") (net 29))
 (segment (start 202.44 95.87) (end 202.44 106.584) (width 0.3) (layer "B.Cu") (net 29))
 (segment (start 200.1725 96.497) (end 200.1725 109.3965) (width 0.4) (layer "B.Cu") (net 30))
 (segment (start 200.1725 109.3965) (end 200.2155 109.4395) (width 0.3) (layer "B.Cu") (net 30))
 (segment (start 214.7225 96.747) (end 225.078 107.1025) (width 1.25) (layer "B.Cu") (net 26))
 (segment (start 225.078 107.1025) (end 226.5125 107.1025) (width 1.25) (layer "B.Cu") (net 26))
 (segment (start 226.5125 102.0225) (end 218.72 94.23) (width 1.25) (layer "B.Cu") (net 25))
 (segment (start 218.72 94.23) (end 214.7395 94.23) (width 1.25) (layer "B.Cu") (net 25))
 (segment (start 214.7395 94.23) (end 214.7225 94.247) (width 1.25) (layer "B.Cu") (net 25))
 (segment (start 221.317 91.747) (end 226.5125 96.9425) (width 1.25) (layer "B.Cu") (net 24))
 (segment (start 214.7225 91.747) (end 221.317 91.747) (width 1.25) (layer "B.Cu") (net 24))
 (segment (start 214.7225 89.247) (end 223.897 89.247) (width 1.25) (layer "B.Cu") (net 23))
 (segment (start 223.897 89.247) (end 226.5125 91.8625) (width 1.25) (layer "B.Cu") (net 23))
 (segment (start 214.7225 86.747) (end 226.477 86.747) (width 1.25) (layer "B.Cu") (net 22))
 (segment (start 226.477 86.747) (end 226.5125 86.7825) (width 1.25) (layer "B.Cu") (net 22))
 (segment (start 214.7225 81.747) (end 226.468 81.747) (width 1.25) (layer "B.Cu") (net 21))
 (segment (start 226.468 81.747) (end 226.5125 81.7025) (width 1.25) (layer "B.Cu") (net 21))
 (segment (start 223.888 79.247) (end 214.7225 79.247) (width 1.25) (layer "B.Cu") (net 20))
 (segment (start 223.888 79.247) (end 226.5125 76.6225) (width 1.25) (layer "B.Cu") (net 20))
 (segment (start 223.808 74.247) (end 226.5125 71.5425) (width 1.25) (layer "B.Cu") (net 19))
 (segment (start 214.7225 74.247) (end 223.808 74.247) (width 1.25) (layer "B.Cu") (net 19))
 (segment (start 214.7225 71.747) (end 221.228 71.747) (width 1.25) (layer "B.Cu") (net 18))
 (segment (start 221.228 71.747) (end 226.5125 66.4625) (width 1.25) (layer "B.Cu") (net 18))
 (segment (start 214.7225 69.247) (end 218.648 69.247) (width 1.25) (layer "B.Cu") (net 17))
 (segment (start 218.648 69.247) (end 226.5125 61.3825) (width 1.25) (layer "B.Cu") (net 17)))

